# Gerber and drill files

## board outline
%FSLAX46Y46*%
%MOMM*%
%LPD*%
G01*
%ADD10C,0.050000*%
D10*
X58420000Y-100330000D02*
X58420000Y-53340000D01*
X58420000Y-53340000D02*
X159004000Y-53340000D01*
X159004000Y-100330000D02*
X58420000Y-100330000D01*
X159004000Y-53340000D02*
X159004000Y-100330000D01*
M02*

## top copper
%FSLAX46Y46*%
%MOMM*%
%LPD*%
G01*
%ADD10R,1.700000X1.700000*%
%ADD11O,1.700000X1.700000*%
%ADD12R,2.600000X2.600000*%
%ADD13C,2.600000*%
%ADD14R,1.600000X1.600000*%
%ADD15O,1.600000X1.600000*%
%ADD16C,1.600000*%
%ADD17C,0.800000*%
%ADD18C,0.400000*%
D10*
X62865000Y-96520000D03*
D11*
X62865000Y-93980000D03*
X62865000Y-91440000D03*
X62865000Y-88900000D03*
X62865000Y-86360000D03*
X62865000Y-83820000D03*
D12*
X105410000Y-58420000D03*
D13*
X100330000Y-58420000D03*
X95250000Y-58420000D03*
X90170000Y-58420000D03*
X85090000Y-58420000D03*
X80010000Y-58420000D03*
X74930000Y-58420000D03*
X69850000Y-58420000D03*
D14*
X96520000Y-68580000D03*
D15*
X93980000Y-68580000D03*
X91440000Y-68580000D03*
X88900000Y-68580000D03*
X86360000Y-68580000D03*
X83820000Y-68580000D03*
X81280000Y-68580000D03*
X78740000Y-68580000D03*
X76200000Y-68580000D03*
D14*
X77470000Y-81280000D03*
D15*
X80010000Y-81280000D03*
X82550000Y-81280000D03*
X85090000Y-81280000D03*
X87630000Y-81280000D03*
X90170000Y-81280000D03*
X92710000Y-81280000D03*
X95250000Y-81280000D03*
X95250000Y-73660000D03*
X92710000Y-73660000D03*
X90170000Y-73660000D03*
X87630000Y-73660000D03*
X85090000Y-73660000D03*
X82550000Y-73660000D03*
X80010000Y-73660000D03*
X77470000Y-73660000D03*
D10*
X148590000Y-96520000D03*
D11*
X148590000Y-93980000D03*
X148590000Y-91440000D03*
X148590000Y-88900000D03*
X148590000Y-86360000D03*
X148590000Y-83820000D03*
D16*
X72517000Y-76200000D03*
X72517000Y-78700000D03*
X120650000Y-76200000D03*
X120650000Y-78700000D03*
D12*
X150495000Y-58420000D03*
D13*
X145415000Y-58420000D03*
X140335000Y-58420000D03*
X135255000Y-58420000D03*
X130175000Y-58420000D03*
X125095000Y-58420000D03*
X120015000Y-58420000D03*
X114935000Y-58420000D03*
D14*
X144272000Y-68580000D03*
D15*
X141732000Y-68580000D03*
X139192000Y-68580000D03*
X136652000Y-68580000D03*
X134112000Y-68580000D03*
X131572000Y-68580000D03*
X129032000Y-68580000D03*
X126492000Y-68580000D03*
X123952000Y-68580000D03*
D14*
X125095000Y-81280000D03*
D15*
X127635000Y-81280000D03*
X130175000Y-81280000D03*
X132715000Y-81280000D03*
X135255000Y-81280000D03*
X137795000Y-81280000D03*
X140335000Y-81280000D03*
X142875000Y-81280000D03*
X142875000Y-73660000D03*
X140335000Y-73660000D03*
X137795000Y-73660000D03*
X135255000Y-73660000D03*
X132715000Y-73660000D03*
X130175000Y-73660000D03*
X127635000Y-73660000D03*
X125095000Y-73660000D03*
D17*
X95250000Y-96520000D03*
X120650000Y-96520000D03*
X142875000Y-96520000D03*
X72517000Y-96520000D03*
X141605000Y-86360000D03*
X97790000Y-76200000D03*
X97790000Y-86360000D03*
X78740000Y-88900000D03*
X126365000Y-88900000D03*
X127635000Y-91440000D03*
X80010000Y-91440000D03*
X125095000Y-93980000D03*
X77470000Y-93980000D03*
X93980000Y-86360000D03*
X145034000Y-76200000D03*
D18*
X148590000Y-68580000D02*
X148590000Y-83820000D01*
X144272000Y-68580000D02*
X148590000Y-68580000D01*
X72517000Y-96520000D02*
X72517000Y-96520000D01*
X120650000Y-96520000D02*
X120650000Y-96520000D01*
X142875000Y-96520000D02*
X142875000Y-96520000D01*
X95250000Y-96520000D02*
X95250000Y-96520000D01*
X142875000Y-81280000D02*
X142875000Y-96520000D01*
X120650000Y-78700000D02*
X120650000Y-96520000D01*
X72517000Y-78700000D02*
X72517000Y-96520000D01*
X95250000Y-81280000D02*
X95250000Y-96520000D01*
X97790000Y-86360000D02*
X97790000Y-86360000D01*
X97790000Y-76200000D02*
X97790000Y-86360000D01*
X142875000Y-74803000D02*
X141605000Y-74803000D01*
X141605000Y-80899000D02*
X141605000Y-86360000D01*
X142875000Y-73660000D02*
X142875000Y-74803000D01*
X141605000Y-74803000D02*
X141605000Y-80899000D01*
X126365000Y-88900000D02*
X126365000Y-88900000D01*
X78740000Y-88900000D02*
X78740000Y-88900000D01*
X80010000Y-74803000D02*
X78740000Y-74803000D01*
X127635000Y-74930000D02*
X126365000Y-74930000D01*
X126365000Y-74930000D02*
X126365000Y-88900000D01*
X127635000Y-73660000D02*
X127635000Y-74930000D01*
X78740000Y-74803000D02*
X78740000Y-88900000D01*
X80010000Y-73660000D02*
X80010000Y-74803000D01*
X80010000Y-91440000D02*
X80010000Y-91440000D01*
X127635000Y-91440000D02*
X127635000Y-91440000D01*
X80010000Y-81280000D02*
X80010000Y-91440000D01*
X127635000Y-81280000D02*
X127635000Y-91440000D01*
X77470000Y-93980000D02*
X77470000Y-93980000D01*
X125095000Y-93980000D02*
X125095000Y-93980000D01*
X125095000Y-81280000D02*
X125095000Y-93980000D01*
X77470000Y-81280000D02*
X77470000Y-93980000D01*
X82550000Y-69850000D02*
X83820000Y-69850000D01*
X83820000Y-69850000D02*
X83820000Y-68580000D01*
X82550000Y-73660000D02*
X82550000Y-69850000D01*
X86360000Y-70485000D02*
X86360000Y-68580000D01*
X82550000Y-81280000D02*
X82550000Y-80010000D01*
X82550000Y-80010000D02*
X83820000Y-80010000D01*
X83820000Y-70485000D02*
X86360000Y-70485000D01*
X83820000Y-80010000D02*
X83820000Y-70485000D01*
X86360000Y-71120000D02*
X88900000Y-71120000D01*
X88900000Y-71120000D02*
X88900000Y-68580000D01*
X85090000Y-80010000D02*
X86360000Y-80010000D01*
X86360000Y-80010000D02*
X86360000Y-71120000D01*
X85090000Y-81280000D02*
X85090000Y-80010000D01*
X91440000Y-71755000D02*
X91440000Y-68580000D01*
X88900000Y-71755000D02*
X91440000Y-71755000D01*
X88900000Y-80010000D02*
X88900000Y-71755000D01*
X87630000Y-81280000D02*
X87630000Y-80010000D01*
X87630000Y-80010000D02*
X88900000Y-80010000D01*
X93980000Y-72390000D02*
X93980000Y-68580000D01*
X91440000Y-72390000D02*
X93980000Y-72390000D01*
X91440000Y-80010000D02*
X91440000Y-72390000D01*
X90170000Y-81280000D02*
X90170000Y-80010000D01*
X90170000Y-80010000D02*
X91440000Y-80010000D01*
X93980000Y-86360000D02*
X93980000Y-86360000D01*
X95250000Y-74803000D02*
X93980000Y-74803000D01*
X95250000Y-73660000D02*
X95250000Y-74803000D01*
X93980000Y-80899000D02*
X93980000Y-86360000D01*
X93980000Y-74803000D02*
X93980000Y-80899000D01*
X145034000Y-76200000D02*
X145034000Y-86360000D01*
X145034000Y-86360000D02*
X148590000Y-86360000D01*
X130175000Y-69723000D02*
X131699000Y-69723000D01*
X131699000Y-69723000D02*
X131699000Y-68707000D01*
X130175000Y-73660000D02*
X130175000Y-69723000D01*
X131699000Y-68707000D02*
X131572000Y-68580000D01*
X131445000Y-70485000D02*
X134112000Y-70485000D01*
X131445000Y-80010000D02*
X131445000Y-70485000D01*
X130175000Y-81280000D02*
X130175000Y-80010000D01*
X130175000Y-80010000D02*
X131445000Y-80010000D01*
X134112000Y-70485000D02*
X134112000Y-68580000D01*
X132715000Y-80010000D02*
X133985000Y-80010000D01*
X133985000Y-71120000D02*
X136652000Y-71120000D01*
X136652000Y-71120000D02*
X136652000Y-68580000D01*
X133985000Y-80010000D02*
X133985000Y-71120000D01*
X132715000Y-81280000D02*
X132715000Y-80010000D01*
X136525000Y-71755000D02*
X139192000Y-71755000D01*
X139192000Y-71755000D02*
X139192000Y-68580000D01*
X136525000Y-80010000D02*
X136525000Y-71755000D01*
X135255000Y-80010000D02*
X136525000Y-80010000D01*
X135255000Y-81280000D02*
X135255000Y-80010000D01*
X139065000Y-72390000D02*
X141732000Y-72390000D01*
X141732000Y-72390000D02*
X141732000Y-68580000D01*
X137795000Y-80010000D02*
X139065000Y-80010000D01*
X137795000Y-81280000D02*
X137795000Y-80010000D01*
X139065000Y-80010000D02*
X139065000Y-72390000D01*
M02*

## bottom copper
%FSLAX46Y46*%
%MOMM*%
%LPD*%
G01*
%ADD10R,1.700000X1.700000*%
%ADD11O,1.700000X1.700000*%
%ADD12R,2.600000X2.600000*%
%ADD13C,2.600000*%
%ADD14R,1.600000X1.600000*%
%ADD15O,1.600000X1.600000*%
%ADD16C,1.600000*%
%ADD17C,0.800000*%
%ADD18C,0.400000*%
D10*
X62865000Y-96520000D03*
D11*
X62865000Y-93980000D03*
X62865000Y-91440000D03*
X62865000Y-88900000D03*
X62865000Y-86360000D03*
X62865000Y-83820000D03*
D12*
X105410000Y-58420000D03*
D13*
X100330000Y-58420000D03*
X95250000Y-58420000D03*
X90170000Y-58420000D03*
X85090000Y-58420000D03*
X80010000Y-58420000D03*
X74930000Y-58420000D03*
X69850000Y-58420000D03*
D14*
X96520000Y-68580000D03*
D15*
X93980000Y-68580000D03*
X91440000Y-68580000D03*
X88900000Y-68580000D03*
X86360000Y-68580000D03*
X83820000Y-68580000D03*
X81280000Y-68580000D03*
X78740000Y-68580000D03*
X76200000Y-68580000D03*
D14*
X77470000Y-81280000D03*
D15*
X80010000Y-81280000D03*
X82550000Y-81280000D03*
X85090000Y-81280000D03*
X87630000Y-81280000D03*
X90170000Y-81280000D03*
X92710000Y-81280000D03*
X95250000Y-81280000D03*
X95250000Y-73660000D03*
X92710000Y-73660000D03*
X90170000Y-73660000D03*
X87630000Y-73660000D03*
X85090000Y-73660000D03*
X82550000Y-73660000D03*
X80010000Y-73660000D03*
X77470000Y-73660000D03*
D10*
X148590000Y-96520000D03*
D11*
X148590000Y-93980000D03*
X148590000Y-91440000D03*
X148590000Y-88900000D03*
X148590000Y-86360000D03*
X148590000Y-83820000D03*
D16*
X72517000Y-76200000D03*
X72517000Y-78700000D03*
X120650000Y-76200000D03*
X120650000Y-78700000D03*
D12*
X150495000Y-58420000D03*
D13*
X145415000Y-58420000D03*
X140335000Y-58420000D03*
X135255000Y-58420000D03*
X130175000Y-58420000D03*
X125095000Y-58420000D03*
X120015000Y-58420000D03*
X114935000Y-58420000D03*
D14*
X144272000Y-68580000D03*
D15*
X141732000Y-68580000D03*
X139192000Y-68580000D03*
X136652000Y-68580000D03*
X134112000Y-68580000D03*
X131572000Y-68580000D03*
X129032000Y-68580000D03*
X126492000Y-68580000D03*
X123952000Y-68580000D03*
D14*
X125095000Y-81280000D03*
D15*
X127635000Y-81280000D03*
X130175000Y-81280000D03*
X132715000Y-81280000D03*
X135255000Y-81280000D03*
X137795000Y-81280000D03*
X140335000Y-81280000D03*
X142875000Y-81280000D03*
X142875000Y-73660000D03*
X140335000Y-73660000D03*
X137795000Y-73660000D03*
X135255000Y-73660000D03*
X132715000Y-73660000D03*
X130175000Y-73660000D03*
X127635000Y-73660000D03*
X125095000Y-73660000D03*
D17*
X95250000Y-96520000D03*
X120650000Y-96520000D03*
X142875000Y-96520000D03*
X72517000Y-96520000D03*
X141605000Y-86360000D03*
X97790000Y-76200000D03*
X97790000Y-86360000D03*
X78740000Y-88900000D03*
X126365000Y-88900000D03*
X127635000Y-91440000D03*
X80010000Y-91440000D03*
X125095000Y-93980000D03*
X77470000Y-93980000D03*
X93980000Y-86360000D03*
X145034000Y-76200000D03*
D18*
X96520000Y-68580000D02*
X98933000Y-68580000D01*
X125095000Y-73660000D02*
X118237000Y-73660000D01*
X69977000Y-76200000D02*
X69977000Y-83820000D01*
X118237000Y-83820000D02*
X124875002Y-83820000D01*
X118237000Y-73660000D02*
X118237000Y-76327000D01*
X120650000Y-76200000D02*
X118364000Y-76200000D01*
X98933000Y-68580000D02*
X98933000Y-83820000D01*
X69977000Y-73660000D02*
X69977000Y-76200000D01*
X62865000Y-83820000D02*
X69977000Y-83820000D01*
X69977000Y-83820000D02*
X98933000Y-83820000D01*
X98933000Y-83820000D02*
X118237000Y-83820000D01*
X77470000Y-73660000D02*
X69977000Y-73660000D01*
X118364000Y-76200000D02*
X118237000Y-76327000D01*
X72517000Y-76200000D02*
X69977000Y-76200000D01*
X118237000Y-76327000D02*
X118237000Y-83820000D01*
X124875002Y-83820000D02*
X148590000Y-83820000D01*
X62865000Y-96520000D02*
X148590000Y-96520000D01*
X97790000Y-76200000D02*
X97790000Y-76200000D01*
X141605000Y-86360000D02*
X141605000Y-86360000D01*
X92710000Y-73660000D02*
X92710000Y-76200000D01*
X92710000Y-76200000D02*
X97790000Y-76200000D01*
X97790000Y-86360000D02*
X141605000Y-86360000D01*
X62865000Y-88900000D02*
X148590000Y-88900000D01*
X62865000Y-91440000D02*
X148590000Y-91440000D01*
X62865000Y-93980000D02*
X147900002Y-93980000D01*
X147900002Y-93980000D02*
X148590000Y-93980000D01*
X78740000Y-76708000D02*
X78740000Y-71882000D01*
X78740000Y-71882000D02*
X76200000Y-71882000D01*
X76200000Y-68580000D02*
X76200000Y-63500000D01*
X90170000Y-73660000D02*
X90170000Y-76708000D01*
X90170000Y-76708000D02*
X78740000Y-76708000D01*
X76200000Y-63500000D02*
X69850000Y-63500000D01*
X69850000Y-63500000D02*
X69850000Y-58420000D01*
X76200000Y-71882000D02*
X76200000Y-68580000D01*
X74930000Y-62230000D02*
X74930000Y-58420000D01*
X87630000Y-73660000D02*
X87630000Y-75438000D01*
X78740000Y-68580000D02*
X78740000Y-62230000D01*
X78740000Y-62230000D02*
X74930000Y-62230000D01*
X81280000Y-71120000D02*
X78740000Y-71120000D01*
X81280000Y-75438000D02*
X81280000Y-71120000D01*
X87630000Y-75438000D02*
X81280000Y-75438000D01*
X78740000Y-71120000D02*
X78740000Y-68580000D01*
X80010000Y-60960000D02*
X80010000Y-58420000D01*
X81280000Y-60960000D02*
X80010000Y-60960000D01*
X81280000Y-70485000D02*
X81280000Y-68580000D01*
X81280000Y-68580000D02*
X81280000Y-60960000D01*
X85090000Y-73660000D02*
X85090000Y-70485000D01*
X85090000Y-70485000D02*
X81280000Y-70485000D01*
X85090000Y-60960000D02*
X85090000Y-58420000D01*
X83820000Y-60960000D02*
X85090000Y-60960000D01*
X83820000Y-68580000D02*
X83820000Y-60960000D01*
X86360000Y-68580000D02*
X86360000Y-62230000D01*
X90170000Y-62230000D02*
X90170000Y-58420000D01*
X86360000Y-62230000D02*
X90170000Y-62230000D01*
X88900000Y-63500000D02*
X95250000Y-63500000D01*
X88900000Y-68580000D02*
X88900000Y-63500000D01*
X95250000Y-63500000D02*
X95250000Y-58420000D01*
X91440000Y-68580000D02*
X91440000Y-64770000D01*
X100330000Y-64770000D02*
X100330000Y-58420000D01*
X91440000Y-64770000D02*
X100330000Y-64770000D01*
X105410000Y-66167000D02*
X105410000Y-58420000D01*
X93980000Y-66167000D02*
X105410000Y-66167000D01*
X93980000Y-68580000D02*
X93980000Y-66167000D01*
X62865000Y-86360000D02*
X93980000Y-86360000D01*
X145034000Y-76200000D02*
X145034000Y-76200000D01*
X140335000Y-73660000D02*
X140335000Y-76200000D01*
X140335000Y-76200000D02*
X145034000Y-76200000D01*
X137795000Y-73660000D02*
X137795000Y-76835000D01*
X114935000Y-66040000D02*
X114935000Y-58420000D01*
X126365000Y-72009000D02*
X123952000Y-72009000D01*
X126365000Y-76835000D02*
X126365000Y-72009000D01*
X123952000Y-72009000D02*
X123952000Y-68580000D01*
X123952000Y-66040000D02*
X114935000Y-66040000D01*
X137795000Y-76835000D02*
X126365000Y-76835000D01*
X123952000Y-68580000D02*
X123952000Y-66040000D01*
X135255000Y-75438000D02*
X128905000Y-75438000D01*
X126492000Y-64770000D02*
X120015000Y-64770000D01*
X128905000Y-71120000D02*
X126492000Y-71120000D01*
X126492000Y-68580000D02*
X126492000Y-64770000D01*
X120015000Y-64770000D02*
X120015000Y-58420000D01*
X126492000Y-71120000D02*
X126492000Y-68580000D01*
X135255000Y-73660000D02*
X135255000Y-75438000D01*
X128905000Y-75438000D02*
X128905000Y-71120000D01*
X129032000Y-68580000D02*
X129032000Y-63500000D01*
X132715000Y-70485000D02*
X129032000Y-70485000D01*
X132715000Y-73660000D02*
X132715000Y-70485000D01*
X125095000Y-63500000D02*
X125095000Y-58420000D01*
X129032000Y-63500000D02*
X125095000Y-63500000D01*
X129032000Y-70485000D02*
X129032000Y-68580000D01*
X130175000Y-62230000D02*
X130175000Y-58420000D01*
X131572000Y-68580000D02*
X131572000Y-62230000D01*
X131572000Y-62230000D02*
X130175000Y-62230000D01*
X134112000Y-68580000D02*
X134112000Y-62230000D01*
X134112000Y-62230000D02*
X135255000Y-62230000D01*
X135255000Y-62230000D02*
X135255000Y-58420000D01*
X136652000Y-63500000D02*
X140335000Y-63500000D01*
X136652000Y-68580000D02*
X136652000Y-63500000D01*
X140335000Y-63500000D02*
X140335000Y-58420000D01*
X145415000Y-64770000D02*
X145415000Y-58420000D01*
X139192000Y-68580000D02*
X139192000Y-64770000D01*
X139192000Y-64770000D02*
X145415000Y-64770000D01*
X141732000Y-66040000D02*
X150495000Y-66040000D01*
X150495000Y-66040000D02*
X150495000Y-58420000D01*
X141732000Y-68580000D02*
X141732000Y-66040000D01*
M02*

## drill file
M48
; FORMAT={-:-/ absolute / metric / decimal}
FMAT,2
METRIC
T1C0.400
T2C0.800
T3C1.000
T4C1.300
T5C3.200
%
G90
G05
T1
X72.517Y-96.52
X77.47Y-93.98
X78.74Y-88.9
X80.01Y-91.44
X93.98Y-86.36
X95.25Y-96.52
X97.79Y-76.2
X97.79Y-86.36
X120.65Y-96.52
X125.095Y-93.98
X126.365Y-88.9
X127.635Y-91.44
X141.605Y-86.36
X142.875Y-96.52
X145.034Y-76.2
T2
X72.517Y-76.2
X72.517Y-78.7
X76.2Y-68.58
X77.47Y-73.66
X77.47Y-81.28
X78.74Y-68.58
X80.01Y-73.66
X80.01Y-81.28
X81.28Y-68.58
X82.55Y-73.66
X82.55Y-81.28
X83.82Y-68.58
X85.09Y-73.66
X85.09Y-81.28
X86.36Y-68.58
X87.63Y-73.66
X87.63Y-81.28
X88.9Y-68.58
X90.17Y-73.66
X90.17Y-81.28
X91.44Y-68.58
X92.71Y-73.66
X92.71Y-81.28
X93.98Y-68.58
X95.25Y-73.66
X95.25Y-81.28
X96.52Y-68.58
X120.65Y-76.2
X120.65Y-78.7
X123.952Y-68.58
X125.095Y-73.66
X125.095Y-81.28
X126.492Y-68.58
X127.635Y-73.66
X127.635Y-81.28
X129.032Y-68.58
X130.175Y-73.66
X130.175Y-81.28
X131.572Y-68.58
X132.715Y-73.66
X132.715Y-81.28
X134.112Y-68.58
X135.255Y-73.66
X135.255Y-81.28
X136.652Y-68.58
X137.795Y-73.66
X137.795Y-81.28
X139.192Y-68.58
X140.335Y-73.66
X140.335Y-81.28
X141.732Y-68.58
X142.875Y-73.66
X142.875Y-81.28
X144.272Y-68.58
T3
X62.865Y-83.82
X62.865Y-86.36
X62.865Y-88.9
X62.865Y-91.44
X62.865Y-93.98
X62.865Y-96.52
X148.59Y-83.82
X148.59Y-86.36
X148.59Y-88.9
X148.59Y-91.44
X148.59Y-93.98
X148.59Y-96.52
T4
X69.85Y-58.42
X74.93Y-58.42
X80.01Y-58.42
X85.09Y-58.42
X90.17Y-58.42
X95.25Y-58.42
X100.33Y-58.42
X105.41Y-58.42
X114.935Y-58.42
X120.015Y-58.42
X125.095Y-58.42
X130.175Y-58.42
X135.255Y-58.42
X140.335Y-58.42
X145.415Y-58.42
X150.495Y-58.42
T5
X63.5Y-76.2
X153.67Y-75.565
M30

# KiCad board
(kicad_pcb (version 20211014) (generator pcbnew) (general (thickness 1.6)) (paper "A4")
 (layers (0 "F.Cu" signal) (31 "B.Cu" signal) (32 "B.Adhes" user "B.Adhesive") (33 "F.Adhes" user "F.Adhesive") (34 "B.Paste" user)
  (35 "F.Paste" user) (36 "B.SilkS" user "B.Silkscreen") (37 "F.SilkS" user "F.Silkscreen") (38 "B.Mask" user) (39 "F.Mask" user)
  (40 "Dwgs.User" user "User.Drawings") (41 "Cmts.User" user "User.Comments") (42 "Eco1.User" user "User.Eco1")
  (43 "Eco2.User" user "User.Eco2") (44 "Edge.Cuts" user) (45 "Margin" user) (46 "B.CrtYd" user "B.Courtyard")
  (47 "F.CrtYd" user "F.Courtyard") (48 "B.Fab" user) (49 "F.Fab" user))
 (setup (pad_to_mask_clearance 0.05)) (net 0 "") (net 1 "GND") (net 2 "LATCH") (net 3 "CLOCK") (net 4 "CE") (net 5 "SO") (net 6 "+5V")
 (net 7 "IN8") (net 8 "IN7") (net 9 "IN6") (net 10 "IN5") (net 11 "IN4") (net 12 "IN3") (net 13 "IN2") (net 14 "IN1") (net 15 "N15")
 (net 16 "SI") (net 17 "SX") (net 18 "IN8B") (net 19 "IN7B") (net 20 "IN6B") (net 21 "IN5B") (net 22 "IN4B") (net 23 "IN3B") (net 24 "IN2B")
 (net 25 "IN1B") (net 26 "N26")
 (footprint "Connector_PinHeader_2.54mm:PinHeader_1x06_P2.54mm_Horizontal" (layer "F.Cu") (at 62.865 96.52 180)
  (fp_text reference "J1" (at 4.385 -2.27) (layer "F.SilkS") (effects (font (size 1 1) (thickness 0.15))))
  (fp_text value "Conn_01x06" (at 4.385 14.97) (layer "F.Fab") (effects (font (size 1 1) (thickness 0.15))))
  (pad "1" thru_hole rect locked (at 0 0 180) (size 1.7 1.7) (drill 1) (layers *.Cu *.Mask) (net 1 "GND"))
  (pad "2" thru_hole oval locked (at 0 2.54 180) (size 1.7 1.7) (drill 1) (layers *.Cu *.Mask) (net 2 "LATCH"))
  (pad "3" thru_hole oval locked (at 0 5.08 180) (size 1.7 1.7) (drill 1) (layers *.Cu *.Mask) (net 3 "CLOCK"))
  (pad "4" thru_hole oval locked (at 0 7.62 180) (size 1.7 1.7) (drill 1) (layers *.Cu *.Mask) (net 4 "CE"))
  (pad "5" thru_hole oval locked (at 0 10.16 180) (size 1.7 1.7) (drill 1) (layers *.Cu *.Mask) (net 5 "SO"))
  (pad "6" thru_hole oval locked (at 0 12.7 180) (size 1.7 1.7) (drill 1) (layers *.Cu *.Mask) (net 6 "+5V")))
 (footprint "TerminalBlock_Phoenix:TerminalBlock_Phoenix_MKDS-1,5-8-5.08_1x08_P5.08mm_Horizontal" (layer "F.Cu") (at 105.41 58.42 180)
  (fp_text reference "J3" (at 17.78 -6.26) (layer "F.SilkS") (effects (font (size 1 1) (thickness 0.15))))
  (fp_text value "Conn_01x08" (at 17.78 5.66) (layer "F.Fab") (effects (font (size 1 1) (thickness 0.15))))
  (pad "1" thru_hole rect locked (at 0 0 180) (size 2.6 2.6) (drill 1.3) (layers *.Cu *.Mask) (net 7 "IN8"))
  (pad "2" thru_hole circle locked (at 5.08 0 180) (size 2.6 2.6) (drill 1.3) (layers *.Cu *.Mask) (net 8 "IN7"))
  (pad "3" thru_hole circle locked (at 10.16 0 180) (size 2.6 2.6) (drill 1.3) (layers *.Cu *.Mask) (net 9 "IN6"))
  (pad "4" thru_hole circle locked (at 15.24 0 180) (size 2.6 2.6) (drill 1.3) (layers *.Cu *.Mask) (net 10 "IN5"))
  (pad "5" thru_hole circle locked (at 20.32 0 180) (size 2.6 2.6) (drill 1.3) (layers *.Cu *.Mask) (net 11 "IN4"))
  (pad "6" thru_hole circle locked (at 25.4 0 180) (size 2.6 2.6) (drill 1.3) (layers *.Cu *.Mask) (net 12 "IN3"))
  (pad "7" thru_hole circle locked (at 30.48 0 180) (size 2.6 2.6) (drill 1.3) (layers *.Cu *.Mask) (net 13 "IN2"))
  (pad "8" thru_hole circle locked (at 35.56 0 180) (size 2.6 2.6) (drill 1.3) (layers *.Cu *.Mask) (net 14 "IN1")))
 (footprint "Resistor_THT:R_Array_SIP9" (layer "F.Cu") (at 96.52 68.58 180)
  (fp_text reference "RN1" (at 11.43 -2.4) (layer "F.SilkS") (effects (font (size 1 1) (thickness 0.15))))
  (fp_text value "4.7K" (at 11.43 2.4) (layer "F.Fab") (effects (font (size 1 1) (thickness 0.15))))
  (pad "1" thru_hole rect locked (at 0 0 180) (size 1.6 1.6) (drill 0.8) (layers *.Cu *.Mask) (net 6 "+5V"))
  (pad "2" thru_hole oval locked (at 2.54 0 180) (size 1.6 1.6) (drill 0.8) (layers *.Cu *.Mask) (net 7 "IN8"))
  (pad "3" thru_hole oval locked (at 5.08 0 180) (size 1.6 1.6) (drill 0.8) (layers *.Cu *.Mask) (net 8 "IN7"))
  (pad "4" thru_hole oval locked (at 7.62 0 180) (size 1.6 1.6) (drill 0.8) (layers *.Cu *.Mask) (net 9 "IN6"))
  (pad "5" thru_hole oval locked (at 10.16 0 180) (size 1.6 1.6) (drill 0.8) (layers *.Cu *.Mask) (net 10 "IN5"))
  (pad "6" thru_hole oval locked (at 12.7 0 180) (size 1.6 1.6) (drill 0.8) (layers *.Cu *.Mask) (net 11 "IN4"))
  (pad "7" thru_hole oval locked (at 15.24 0 180) (size 1.6 1.6) (drill 0.8) (layers *.Cu *.Mask) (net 12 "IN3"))
  (pad "8" thru_hole oval locked (at 17.78 0 180) (size 1.6 1.6) (drill 0.8) (layers *.Cu *.Mask) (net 13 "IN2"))
  (pad "9" thru_hole oval locked (at 20.32 0 180) (size 1.6 1.6) (drill 0.8) (layers *.Cu *.Mask) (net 14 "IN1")))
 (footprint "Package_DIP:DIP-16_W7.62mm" (layer "F.Cu") (at 77.47 81.28 90)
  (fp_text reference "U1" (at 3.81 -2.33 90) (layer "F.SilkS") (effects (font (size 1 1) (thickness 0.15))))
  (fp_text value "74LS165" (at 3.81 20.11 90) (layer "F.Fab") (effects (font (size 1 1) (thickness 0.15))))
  (pad "1" thru_hole rect locked (at 0 0 90) (size 1.6 1.6) (drill 0.8) (layers *.Cu *.Mask) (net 2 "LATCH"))
  (pad "2" thru_hole oval locked (at 0 2.54 90) (size 1.6 1.6) (drill 0.8) (layers *.Cu *.Mask) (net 3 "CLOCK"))
  (pad "3" thru_hole oval locked (at 0 5.08 90) (size 1.6 1.6) (drill 0.8) (layers *.Cu *.Mask) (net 10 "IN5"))
  (pad "4" thru_hole oval locked (at 0 7.62 90) (size 1.6 1.6) (drill 0.8) (layers *.Cu *.Mask) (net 9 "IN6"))
  (pad "5" thru_hole oval locked (at 0 10.16 90) (size 1.6 1.6) (drill 0.8) (layers *.Cu *.Mask) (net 8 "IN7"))
  (pad "6" thru_hole oval locked (at 0 12.7 90) (size 1.6 1.6) (drill 0.8) (layers *.Cu *.Mask) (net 7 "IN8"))
  (pad "7" thru_hole oval locked (at 0 15.24 90) (size 1.6 1.6) (drill 0.8) (layers *.Cu *.Mask) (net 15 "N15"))
  (pad "8" thru_hole oval locked (at 0 17.78 90) (size 1.6 1.6) (drill 0.8) (layers *.Cu *.Mask) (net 1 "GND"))
  (pad "9" thru_hole oval locked (at 7.62 17.78 90) (size 1.6 1.6) (drill 0.8) (layers *.Cu *.Mask) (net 5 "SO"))
  (pad "10" thru_hole oval locked (at 7.62 15.24 90) (size 1.6 1.6) (drill 0.8) (layers *.Cu *.Mask) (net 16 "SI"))
  (pad "11" thru_hole oval locked (at 7.62 12.7 90) (size 1.6 1.6) (drill 0.8) (layers *.Cu *.Mask) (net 14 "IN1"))
  (pad "12" thru_hole oval locked (at 7.62 10.16 90) (size 1.6 1.6) (drill 0.8) (layers *.Cu *.Mask) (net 13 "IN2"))
  (pad "13" thru_hole oval locked (at 7.62 7.62 90) (size 1.6 1.6) (drill 0.8) (layers *.Cu *.Mask) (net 12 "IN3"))
  (pad "14" thru_hole oval locked (at 7.62 5.08 90) (size 1.6 1.6) (drill 0.8) (layers *.Cu *.Mask) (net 11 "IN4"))
  (pad "15" thru_hole oval locked (at 7.62 2.54 90) (size 1.6 1.6) (drill 0.8) (layers *.Cu *.Mask) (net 4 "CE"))
  (pad "16" thru_hole oval locked (at 7.62 0 90) (size 1.6 1.6) (drill 0.8) (layers *.Cu *.Mask) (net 6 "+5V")))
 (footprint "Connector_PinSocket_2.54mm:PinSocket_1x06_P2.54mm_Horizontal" (layer "F.Cu") (at 148.59 96.52 180)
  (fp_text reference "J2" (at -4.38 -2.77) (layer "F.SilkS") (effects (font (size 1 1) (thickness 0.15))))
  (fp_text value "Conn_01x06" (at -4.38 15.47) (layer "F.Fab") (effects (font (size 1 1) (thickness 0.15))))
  (pad "1" thru_hole rect locked (at 0 0 180) (size 1.7 1.7) (drill 1) (layers *.Cu *.Mask) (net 1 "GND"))
  (pad "2" thru_hole oval locked (at 0 2.54 180) (size 1.7 1.7) (drill 1) (layers *.Cu *.Mask) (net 2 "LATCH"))
  (pad "3" thru_hole oval locked (at 0 5.08 180) (size 1.7 1.7) (drill 1) (layers *.Cu *.Mask) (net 3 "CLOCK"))
  (pad "4" thru_hole oval locked (at 0 7.62 180) (size 1.7 1.7) (drill 1) (layers *.Cu *.Mask) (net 4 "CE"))
  (pad "5" thru_hole oval locked (at 0 10.16 180) (size 1.7 1.7) (drill 1) (layers *.Cu *.Mask) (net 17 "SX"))
  (pad "6" thru_hole oval locked (at 0 12.7 180) (size 1.7 1.7) (drill 1) (layers *.Cu *.Mask) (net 6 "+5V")))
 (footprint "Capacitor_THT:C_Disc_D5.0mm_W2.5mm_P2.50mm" (layer "F.Cu") (at 72.517 76.2 -90)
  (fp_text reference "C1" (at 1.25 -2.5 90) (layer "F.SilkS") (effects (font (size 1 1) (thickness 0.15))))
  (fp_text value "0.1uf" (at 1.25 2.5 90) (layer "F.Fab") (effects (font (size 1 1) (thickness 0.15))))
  (pad "1" thru_hole circle locked (at 0 0 270) (size 1.6 1.6) (drill 0.8) (layers *.Cu *.Mask) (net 6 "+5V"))
  (pad "2" thru_hole circle locked (at 2.5 0 270) (size 1.6 1.6) (drill 0.8) (layers *.Cu *.Mask) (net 1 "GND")))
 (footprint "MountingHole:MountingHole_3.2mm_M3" (layer "F.Cu") (at 153.67 75.565)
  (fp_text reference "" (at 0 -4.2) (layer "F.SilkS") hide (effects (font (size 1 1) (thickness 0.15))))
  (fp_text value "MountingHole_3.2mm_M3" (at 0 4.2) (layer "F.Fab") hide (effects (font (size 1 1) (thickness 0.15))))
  (pad "" np_thru_hole circle locked (at 0 0) (size 3.2 3.2) (drill 3.2) (layers *.Cu *.Mask)))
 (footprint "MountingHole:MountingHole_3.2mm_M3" (layer "F.Cu") (at 63.5 76.2)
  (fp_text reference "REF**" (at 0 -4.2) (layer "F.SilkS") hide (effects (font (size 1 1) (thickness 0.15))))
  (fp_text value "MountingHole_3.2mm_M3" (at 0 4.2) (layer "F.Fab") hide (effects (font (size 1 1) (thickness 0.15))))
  (pad "" np_thru_hole circle locked (at 0 0) (size 3.2 3.2) (drill 3.2) (layers *.Cu *.Mask)))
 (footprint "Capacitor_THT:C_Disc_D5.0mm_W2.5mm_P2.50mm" (layer "F.Cu") (at 120.65 76.2 -90)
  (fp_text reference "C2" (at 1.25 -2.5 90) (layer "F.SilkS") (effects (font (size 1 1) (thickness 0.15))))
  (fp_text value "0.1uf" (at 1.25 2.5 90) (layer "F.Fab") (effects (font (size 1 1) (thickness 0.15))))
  (pad "1" thru_hole circle locked (at 0 0 270) (size 1.6 1.6) (drill 0.8) (layers *.Cu *.Mask) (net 6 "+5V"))
  (pad "2" thru_hole circle locked (at 2.5 0 270) (size 1.6 1.6) (drill 0.8) (layers *.Cu *.Mask) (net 1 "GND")))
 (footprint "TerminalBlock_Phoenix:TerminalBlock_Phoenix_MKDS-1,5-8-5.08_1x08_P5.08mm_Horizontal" (layer "F.Cu") (at 150.495 58.42 180)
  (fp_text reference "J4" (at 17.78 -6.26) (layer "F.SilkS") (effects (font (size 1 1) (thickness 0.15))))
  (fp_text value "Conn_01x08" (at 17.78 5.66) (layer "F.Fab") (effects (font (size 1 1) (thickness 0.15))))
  (pad "1" thru_hole rect locked (at 0 0 180) (size 2.6 2.6) (drill 1.3) (layers *.Cu *.Mask) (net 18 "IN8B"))
  (pad "2" thru_hole circle locked (at 5.08 0 180) (size 2.6 2.6) (drill 1.3) (layers *.Cu *.Mask) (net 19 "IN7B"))
  (pad "3" thru_hole circle locked (at 10.16 0 180) (size 2.6 2.6) (drill 1.3) (layers *.Cu *.Mask) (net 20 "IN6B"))
  (pad "4" thru_hole circle locked (at 15.24 0 180) (size 2.6 2.6) (drill 1.3) (layers *.Cu *.Mask) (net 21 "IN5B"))
  (pad "5" thru_hole circle locked (at 20.32 0 180) (size 2.6 2.6) (drill 1.3) (layers *.Cu *.Mask) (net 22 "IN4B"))
  (pad "6" thru_hole circle locked (at 25.4 0 180) (size 2.6 2.6) (drill 1.3) (layers *.Cu *.Mask) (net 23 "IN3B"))
  (pad "7" thru_hole circle locked (at 30.48 0 180) (size 2.6 2.6) (drill 1.3) (layers *.Cu *.Mask) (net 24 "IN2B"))
  (pad "8" thru_hole circle locked (at 35.56 0 180) (size 2.6 2.6) (drill 1.3) (layers *.Cu *.Mask) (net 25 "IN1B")))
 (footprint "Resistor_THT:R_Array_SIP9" (layer "F.Cu") (at 144.272 68.58 180)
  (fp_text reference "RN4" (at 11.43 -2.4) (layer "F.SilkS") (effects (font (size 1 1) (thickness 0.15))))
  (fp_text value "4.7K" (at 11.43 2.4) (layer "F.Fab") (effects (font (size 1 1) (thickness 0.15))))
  (pad "1" thru_hole rect locked (at 0 0 180) (size 1.6 1.6) (drill 0.8) (layers *.Cu *.Mask) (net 6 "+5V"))
  (pad "2" thru_hole oval locked (at 2.54 0 180) (size 1.6 1.6) (drill 0.8) (layers *.Cu *.Mask) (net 18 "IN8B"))
  (pad "3" thru_hole oval locked (at 5.08 0 180) (size 1.6 1.6) (drill 0.8) (layers *.Cu *.Mask) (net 19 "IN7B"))
  (pad "4" thru_hole oval locked (at 7.62 0 180) (size 1.6 1.6) (drill 0.8) (layers *.Cu *.Mask) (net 20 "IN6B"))
  (pad "5" thru_hole oval locked (at 10.16 0 180) (size 1.6 1.6) (drill 0.8) (layers *.Cu *.Mask) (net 21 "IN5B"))
  (pad "6" thru_hole oval locked (at 12.7 0 180) (size 1.6 1.6) (drill 0.8) (layers *.Cu *.Mask) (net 22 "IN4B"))
  (pad "7" thru_hole oval locked (at 15.24 0 180) (size 1.6 1.6) (drill 0.8) (layers *.Cu *.Mask) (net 23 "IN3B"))
  (pad "8" thru_hole oval locked (at 17.78 0 180) (size 1.6 1.6) (drill 0.8) (layers *.Cu *.Mask) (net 24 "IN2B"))
  (pad "9" thru_hole oval locked (at 20.32 0 180) (size 1.6 1.6) (drill 0.8) (layers *.Cu *.Mask) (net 25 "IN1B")))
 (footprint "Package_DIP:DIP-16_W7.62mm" (layer "F.Cu") (at 125.095 81.28 90)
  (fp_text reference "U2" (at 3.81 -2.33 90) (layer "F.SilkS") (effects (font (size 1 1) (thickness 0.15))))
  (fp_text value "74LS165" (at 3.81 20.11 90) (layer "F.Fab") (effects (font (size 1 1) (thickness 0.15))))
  (pad "1" thru_hole rect locked (at 0 0 90) (size 1.6 1.6) (drill 0.8) (layers *.Cu *.Mask) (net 2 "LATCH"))
  (pad "2" thru_hole oval locked (at 0 2.54 90) (size 1.6 1.6) (drill 0.8) (layers *.Cu *.Mask) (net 3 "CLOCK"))
  (pad "3" thru_hole oval locked (at 0 5.08 90) (size 1.6 1.6) (drill 0.8) (layers *.Cu *.Mask) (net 21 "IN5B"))
  (pad "4" thru_hole oval locked (at 0 7.62 90) (size 1.6 1.6) (drill 0.8) (layers *.Cu *.Mask) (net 20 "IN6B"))
  (pad "5" thru_hole oval locked (at 0 10.16 90) (size 1.6 1.6) (drill 0.8) (layers *.Cu *.Mask) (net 19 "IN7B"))
  (pad "6" thru_hole oval locked (at 0 12.7 90) (size 1.6 1.6) (drill 0.8) (layers *.Cu *.Mask) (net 18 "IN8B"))
  (pad "7" thru_hole oval locked (at 0 15.24 90) (size 1.6 1.6) (drill 0.8) (layers *.Cu *.Mask) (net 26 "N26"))
  (pad "8" thru_hole oval locked (at 0 17.78 90) (size 1.6 1.6) (drill 0.8) (layers *.Cu *.Mask) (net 1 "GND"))
  (pad "9" thru_hole oval locked (at 7.62 17.78 90) (size 1.6 1.6) (drill 0.8) (layers *.Cu *.Mask) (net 16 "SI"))
  (pad "10" thru_hole oval locked (at 7.62 15.24 90) (size 1.6 1.6) (drill 0.8) (layers *.Cu *.Mask) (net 17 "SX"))
  (pad "11" thru_hole oval locked (at 7.62 12.7 90) (size 1.6 1.6) (drill 0.8) (layers *.Cu *.Mask) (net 25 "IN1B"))
  (pad "12" thru_hole oval locked (at 7.62 10.16 90) (size 1.6 1.6) (drill 0.8) (layers *.Cu *.Mask) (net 24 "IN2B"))
  (pad "13" thru_hole oval locked (at 7.62 7.62 90) (size 1.6 1.6) (drill 0.8) (layers *.Cu *.Mask) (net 23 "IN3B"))
  (pad "14" thru_hole oval locked (at 7.62 5.08 90) (size 1.6 1.6) (drill 0.8) (layers *.Cu *.Mask) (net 22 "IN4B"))
  (pad "15" thru_hole oval locked (at 7.62 2.54 90) (size 1.6 1.6) (drill 0.8) (layers *.Cu *.Mask) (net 4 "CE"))
  (pad "16" thru_hole oval locked (at 7.62 0 90) (size 1.6 1.6) (drill 0.8) (layers *.Cu *.Mask) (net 6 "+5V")))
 (gr_line (start 58.42 100.33) (end 58.42 53.34) (layer "Edge.Cuts") (width 0.05))
 (gr_line (start 58.42 53.34) (end 159.004 53.34) (layer "Edge.Cuts") (width 0.05))
 (gr_line (start 159.004 100.33) (end 58.42 100.33) (layer "Edge.Cuts") (width 0.05))
 (gr_line (start 159.004 53.34) (end 159.004 100.33) (layer "Edge.Cuts") (width 0.05))
 (segment (start 148.59 68.58) (end 148.59 83.82) (width 0.4) (layer "F.Cu") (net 6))
 (segment (start 144.272 68.58) (end 148.59 68.58) (width 0.4) (layer "F.Cu") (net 6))
 (segment (start 96.52 68.58) (end 98.933 68.58) (width 0.4) (layer "B.Cu") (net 6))
 (segment (start 125.095 73.66) (end 118.237 73.66) (width 0.4) (layer "B.Cu") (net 6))
 (segment (start 69.977 76.2) (end 69.977 83.82) (width 0.4) (layer "B.Cu") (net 6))
 (segment (start 118.237 83.82) (end 124.875002 83.82) (width 0.4) (layer "B.Cu") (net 6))
 (segment (start 118.237 73.66) (end 118.237 76.327) (width 0.4) (layer "B.Cu") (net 6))
 (segment (start 120.65 76.2) (end 118.364 76.2) (width 0.4) (layer "B.Cu") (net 6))
 (segment (start 98.933 68.58) (end 98.933 83.82) (width 0.4) (layer "B.Cu") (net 6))
 (segment (start 69.977 73.66) (end 69.977 76.2) (width 0.4) (layer "B.Cu") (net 6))
 (segment (start 62.865 83.82) (end 69.977 83.82) (width 0.4) (layer "B.Cu") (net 6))
 (segment (start 69.977 83.82) (end 98.933 83.82) (width 0.4) (layer "B.Cu") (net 6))
 (segment (start 98.933 83.82) (end 118.237 83.82) (width 0.4) (layer "B.Cu") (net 6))
 (segment (start 77.47 73.66) (end 69.977 73.66) (width 0.4) (layer "B.Cu") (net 6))
 (segment (start 118.364 76.2) (end 118.237 76.327) (width 0.4) (layer "B.Cu") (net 6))
 (segment (start 72.517 76.2) (end 69.977 76.2) (width 0.4) (layer "B.Cu") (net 6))
 (segment (start 118.237 76.327) (end 118.237 83.82) (width 0.4) (layer "B.Cu") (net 6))
 (segment (start 124.875002 83.82) (end 148.59 83.82) (width 0.4) (layer "B.Cu") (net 6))
 (segment (start 72.517 96.52) (end 72.517 96.52) (width 0.4) (layer "F.Cu") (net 1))
 (segment (start 120.65 96.52) (end 120.65 96.52) (width 0.4) (layer "F.Cu") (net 1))
 (segment (start 142.875 96.52) (end 142.875 96.52) (width 0.4) (layer "F.Cu") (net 1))
 (segment (start 95.25 96.52) (end 95.25 96.52) (width 0.4) (layer "F.Cu") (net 1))
 (segment (start 142.875 81.28) (end 142.875 96.52) (width 0.4) (layer "F.Cu") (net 1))
 (segment (start 120.65 78.7) (end 120.65 96.52) (width 0.4) (layer "F.Cu") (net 1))
 (segment (start 72.517 78.7) (end 72.517 96.52) (width 0.4) (layer "F.Cu") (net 1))
 (segment (start 95.25 81.28) (end 95.25 96.52) (width 0.4) (layer "F.Cu") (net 1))
 (via (at 95.25 96.52) (size 0.8) (drill 0.4) (layers "F.Cu" "B.Cu") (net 1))
 (via (at 120.65 96.52) (size 0.8) (drill 0.4) (layers "F.Cu" "B.Cu") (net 1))
 (via (at 142.875 96.52) (size 0.8) (drill 0.4) (layers "F.Cu" "B.Cu") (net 1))
 (via (at 72.517 96.52) (size 0.8) (drill 0.4) (layers "F.Cu" "B.Cu") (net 1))
 (segment (start 62.865 96.52) (end 148.59 96.52) (width 0.4) (layer "B.Cu") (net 1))
 (segment (start 97.79 86.36) (end 97.79 86.36) (width 0.4) (layer "F.Cu") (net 16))
 (segment (start 97.79 76.2) (end 97.79 86.36) (width 0.4) (layer "F.Cu") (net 16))
 (segment (start 142.875 74.803) (end 141.605 74.803) (width 0.4) (layer "F.Cu") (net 16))
 (segment (start 141.605 80.899) (end 141.605 86.36) (width 0.4) (layer "F.Cu") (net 16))
 (segment (start 142.875 73.66) (end 142.875 74.803) (width 0.4) (layer "F.Cu") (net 16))
 (segment (start 141.605 74.803) (end 141.605 80.899) (width 0.4) (layer "F.Cu") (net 16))
 (via (at 141.605 86.36) (size 0.8) (drill 0.4) (layers "F.Cu" "B.Cu") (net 16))
 (via (at 97.79 76.2) (size 0.8) (drill 0.4) (layers "F.Cu" "B.Cu") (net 16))
 (via (at 97.79 86.36) (size 0.8) (drill 0.4) (layers "F.Cu" "B.Cu") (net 16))
 (segment (start 97.79 76.2) (end 97.79 76.2) (width 0.4) (layer "B.Cu") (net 16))
 (segment (start 141.605 86.36) (end 141.605 86.36) (width 0.4) (layer "B.Cu") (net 16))
 (segment (start 92.71 73.66) (end 92.71 76.2) (width 0.4) (layer "B.Cu") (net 16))
 (segment (start 92.71 76.2) (end 97.79 76.2) (width 0.4) (layer "B.Cu") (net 16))
 (segment (start 97.79 86.36) (end 141.605 86.36) (width 0.4) (layer "B.Cu") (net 16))
 (segment (start 126.365 88.9) (end 126.365 88.9) (width 0.4) (layer "F.Cu") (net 4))
 (segment (start 78.74 88.9) (end 78.74 88.9) (width 0.4) (layer "F.Cu") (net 4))
 (segment (start 80.01 74.803) (end 78.74 74.803) (width 0.4) (layer "F.Cu") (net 4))
 (segment (start 127.635 74.93) (end 126.365 74.93) (width 0.4) (layer "F.Cu") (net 4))
 (segment (start 126.365 74.93) (end 126.365 88.9) (width 0.4) (layer "F.Cu") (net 4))
 (segment (start 127.635 73.66) (end 127.635 74.93) (width 0.4) (layer "F.Cu") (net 4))
 (segment (start 78.74 74.803) (end 78.74 88.9) (width 0.4) (layer "F.Cu") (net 4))
 (segment (start 80.01 73.66) (end 80.01 74.803) (width 0.4) (layer "F.Cu") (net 4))
 (via (at 78.74 88.9) (size 0.8) (drill 0.4) (layers "F.Cu" "B.Cu") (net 4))
 (via (at 126.365 88.9) (size 0.8) (drill 0.4) (layers "F.Cu" "B.Cu") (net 4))
 (segment (start 62.865 88.9) (end 148.59 88.9) (width 0.4) (layer "B.Cu") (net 4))
 (segment (start 80.01 91.44) (end 80.01 91.44) (width 0.4) (layer "F.Cu") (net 3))
 (segment (start 127.635 91.44) (end 127.635 91.44) (width 0.4) (layer "F.Cu") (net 3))
 (segment (start 80.01 81.28) (end 80.01 91.44) (width 0.4) (layer "F.Cu") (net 3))
 (segment (start 127.635 81.28) (end 127.635 91.44) (width 0.4) (layer "F.Cu") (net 3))
 (via (at 127.635 91.44) (size 0.8) (drill 0.4) (layers "F.Cu" "B.Cu") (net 3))
 (via (at 80.01 91.44) (size 0.8) (drill 0.4) (layers "F.Cu" "B.Cu") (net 3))
 (segment (start 62.865 91.44) (end 148.59 91.44) (width 0.4) (layer "B.Cu") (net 3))
 (segment (start 77.47 93.98) (end 77.47 93.98) (width 0.4) (layer "F.Cu") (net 2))
 (segment (start 125.095 93.98) (end 125.095 93.98) (width 0.4) (layer "F.Cu") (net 2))
 (segment (start 125.095 81.28) (end 125.095 93.98) (width 0.4) (layer "F.Cu") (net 2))
 (segment (start 77.47 81.28) (end 77.47 93.98) (width 0.4) (layer "F.Cu") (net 2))
 (via (at 125.095 93.98) (size 0.8) (drill 0.4) (layers "F.Cu" "B.Cu") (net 2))
 (via (at 77.47 93.98) (size 0.8) (drill 0.4) (layers "F.Cu" "B.Cu") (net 2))
 (segment (start 62.865 93.98) (end 147.900002 93.98) (width 0.4) (layer "B.Cu") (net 2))
 (segment (start 147.900002 93.98) (end 148.59 93.98) (width 0.4) (layer "B.Cu") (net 2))
 (segment (start 78.74 76.708) (end 78.74 71.882) (width 0.4) (layer "B.Cu") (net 14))
 (segment (start 78.74 71.882) (end 76.2 71.882) (width 0.4) (layer "B.Cu") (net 14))
 (segment (start 76.2 68.58) (end 76.2 63.5) (width 0.4) (layer "B.Cu") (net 14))
 (segment (start 90.17 73.66) (end 90.17 76.708) (width 0.4) (layer "B.Cu") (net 14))
 (segment (start 90.17 76.708) (end 78.74 76.708) (width 0.4) (layer "B.Cu") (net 14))
 (segment (start 76.2 63.5) (end 69.85 63.5) (width 0.4) (layer "B.Cu") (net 14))
 (segment (start 69.85 63.5) (end 69.85 58.42) (width 0.4) (layer "B.Cu") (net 14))
 (segment (start 76.2 71.882) (end 76.2 68.58) (width 0.4) (layer "B.Cu") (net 14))
 (segment (start 74.93 62.23) (end 74.93 58.42) (width 0.4) (layer "B.Cu") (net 13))
 (segment (start 87.63 73.66) (end 87.63 75.438) (width 0.4) (layer "B.Cu") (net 13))
 (segment (start 78.74 68.58) (end 78.74 62.23) (width 0.4) (layer "B.Cu") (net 13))
 (segment (start 78.74 62.23) (end 74.93 62.23) (width 0.4) (layer "B.Cu") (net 13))
 (segment (start 81.28 71.12) (end 78.74 71.12) (width 0.4) (layer "B.Cu") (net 13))
 (segment (start 81.28 75.438) (end 81.28 71.12) (width 0.4) (layer "B.Cu") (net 13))
 (segment (start 87.63 75.438) (end 81.28 75.438) (width 0.4) (layer "B.Cu") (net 13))
 (segment (start 78.74 71.12) (end 78.74 68.58) (width 0.4) (layer "B.Cu") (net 13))
 (segment (start 80.01 60.96) (end 80.01 58.42) (width 0.4) (layer "B.Cu") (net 12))
 (segment (start 81.28 60.96) (end 80.01 60.96) (width 0.4) (layer "B.Cu") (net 12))
 (segment (start 81.28 70.485) (end 81.28 68.58) (width 0.4) (layer "B.Cu") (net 12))
 (segment (start 81.28 68.58) (end 81.28 60.96) (width 0.4) (layer "B.Cu") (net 12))
 (segment (start 85.09 73.66) (end 85.09 70.485) (width 0.4) (layer "B.Cu") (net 12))
 (segment (start 85.09 70.485) (end 81.28 70.485) (width 0.4) (layer "B.Cu") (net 12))
 (segment (start 82.55 69.85) (end 83.82 69.85) (width 0.4) (layer "F.Cu") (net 11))
 (segment (start 83.82 69.85) (end 83.82 68.58) (width 0.4) (layer "F.Cu") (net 11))
 (segment (start 82.55 73.66) (end 82.55 69.85) (width 0.4) (layer "F.Cu") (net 11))
 (segment (start 85.09 60.96) (end 85.09 58.42) (width 0.4) (layer "B.Cu") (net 11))
 (segment (start 83.82 60.96) (end 85.09 60.96) (width 0.4) (layer "B.Cu") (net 11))
 (segment (start 83.82 68.58) (end 83.82 60.96) (width 0.4) (layer "B.Cu") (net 11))
 (segment (start 86.36 70.485) (end 86.36 68.58) (width 0.4) (layer "F.Cu") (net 10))
 (segment (start 82.55 81.28) (end 82.55 80.01) (width 0.4) (layer "F.Cu") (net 10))
 (segment (start 82.55 80.01) (end 83.82 80.01) (width 0.4) (layer "F.Cu") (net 10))
 (segment (start 83.82 70.485) (end 86.36 70.485) (width 0.4) (layer "F.Cu") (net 10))
 (segment (start 83.82 80.01) (end 83.82 70.485) (width 0.4) (layer "F.Cu") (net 10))
 (segment (start 86.36 68.58) (end 86.36 62.23) (width 0.4) (layer "B.Cu") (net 10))
 (segment (start 90.17 62.23) (end 90.17 58.42) (width 0.4) (layer "B.Cu") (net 10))
 (segment (start 86.36 62.23) (end 90.17 62.23) (width 0.4) (layer "B.Cu") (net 10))
 (segment (start 86.36 71.12) (end 88.9 71.12) (width 0.4) (layer "F.Cu") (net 9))
 (segment (start 88.9 71.12) (end 88.9 68.58) (width 0.4) (layer "F.Cu") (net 9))
 (segment (start 85.09 80.01) (end 86.36 80.01) (width 0.4) (layer "F.Cu") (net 9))
 (segment (start 86.36 80.01) (end 86.36 71.12) (width 0.4) (layer "F.Cu") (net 9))
 (segment (start 85.09 81.28) (end 85.09 80.01) (width 0.4) (layer "F.Cu") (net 9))
 (segment (start 88.9 63.5) (end 95.25 63.5) (width 0.4) (layer "B.Cu") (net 9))
 (segment (start 88.9 68.58) (end 88.9 63.5) (width 0.4) (layer "B.Cu") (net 9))
 (segment (start 95.25 63.5) (end 95.25 58.42) (width 0.4) (layer "B.Cu") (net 9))
 (segment (start 91.44 71.755) (end 91.44 68.58) (width 0.4) (layer "F.Cu") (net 8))
 (segment (start 88.9 71.755) (end 91.44 71.755) (width 0.4) (layer "F.Cu") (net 8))
 (segment (start 88.9 80.01) (end 88.9 71.755) (width 0.4) (layer "F.Cu") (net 8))
 (segment (start 87.63 81.28) (end 87.63 80.01) (width 0.4) (layer "F.Cu") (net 8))
 (segment (start 87.63 80.01) (end 88.9 80.01) (width 0.4) (layer "F.Cu") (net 8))
 (segment (start 91.44 68.58) (end 91.44 64.77) (width 0.4) (layer "B.Cu") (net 8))
 (segment (start 100.33 64.77) (end 100.33 58.42) (width 0.4) (layer "B.Cu") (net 8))
 (segment (start 91.44 64.77) (end 100.33 64.77) (width 0.4) (layer "B.Cu") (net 8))
 (segment (start 93.98 72.39) (end 93.98 68.58) (width 0.4) (layer "F.Cu") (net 7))
 (segment (start 91.44 72.39) (end 93.98 72.39) (width 0.4) (layer "F.Cu") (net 7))
 (segment (start 91.44 80.01) (end 91.44 72.39) (width 0.4) (layer "F.Cu") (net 7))
 (segment (start 90.17 81.28) (end 90.17 80.01) (width 0.4) (layer "F.Cu") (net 7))
 (segment (start 90.17 80.01) (end 91.44 80.01) (width 0.4) (layer "F.Cu") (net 7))
 (segment (start 105.41 66.167) (end 105.41 58.42) (width 0.4) (layer "B.Cu") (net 7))
 (segment (start 93.98 66.167) (end 105.41 66.167) (width 0.4) (layer "B.Cu") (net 7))
 (segment (start 93.98 68.58) (end 93.98 66.167) (width 0.4) (layer "B.Cu") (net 7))
 (segment (start 93.98 86.36) (end 93.98 86.36) (width 0.4) (layer "F.Cu") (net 5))
 (segment (start 95.25 74.803) (end 93.98 74.803) (width 0.4) (layer "F.Cu") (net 5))
 (segment (start 95.25 73.66) (end 95.25 74.803) (width 0.4) (layer "F.Cu") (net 5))
 (segment (start 93.98 80.899) (end 93.98 86.36) (width 0.4) (layer "F.Cu") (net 5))
 (segment (start 93.98 74.803) (end 93.98 80.899) (width 0.4) (layer "F.Cu") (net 5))
 (via (at 93.98 86.36) (size 0.8) (drill 0.4) (layers "F.Cu" "B.Cu") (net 5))
 (segment (start 62.865 86.36) (end 93.98 86.36) (width 0.4) (layer "B.Cu") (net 5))
 (segment (start 145.034 76.2) (end 145.034 86.36) (width 0.4) (layer "F.Cu") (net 17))
 (segment (start 145.034 86.36) (end 148.59 86.36) (width 0.4) (layer "F.Cu") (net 17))
 (via (at 145.034 76.2) (size 0.8) (drill 0.4) (layers "F.Cu" "B.Cu") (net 17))
 (segment (start 145.034 76.2) (end 145.034 76.2) (width 0.4) (layer "B.Cu") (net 17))
 (segment (start 140.335 73.66) (end 140.335 76.2) (width 0.4) (layer "B.Cu") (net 17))
 (segment (start 140.335 76.2) (end 145.034 76.2) (width 0.4) (layer "B.Cu") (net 17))
 (segment (start 137.795 73.66) (end 137.795 76.835) (width 0.4) (layer "B.Cu") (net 25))
 (segment (start 114.935 66.04) (end 114.935 58.42) (width 0.4) (layer "B.Cu") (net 25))
 (segment (start 126.365 72.009) (end 123.952 72.009) (width 0.4) (layer "B.Cu") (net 25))
 (segment (start 126.365 76.835) (end 126.365 72.009) (width 0.4) (layer "B.Cu") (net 25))
 (segment (start 123.952 72.009) (end 123.952 68.58) (width 0.4) (layer "B.Cu") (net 25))
 (segment (start 123.952 66.04) (end 114.935 66.04) (width 0.4) (layer "B.Cu") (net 25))
 (segment (start 137.795 76.835) (end 126.365 76.835) (width 0.4) (layer "B.Cu") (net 25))
 (segment (start 123.952 68.58) (end 123.952 66.04) (width 0.4) (layer "B.Cu") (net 25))
 (segment (start 135.255 75.438) (end 128.905 75.438) (width 0.4) (layer "B.Cu") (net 24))
 (segment (start 126.492 64.77) (end 120.015 64.77) (width 0.4) (layer "B.Cu") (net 24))
 (segment (start 128.905 71.12) (end 126.492 71.12) (width 0.4) (layer "B.Cu") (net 24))
 (segment (start 126.492 68.58) (end 126.492 64.77) (width 0.4) (layer "B.Cu") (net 24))
 (segment (start 120.015 64.77) (end 120.015 58.42) (width 0.4) (layer "B.Cu") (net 24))
 (segment (start 126.492 71.12) (end 126.492 68.58) (width 0.4) (layer "B.Cu") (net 24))
 (segment (start 135.255 73.66) (end 135.255 75.438) (width 0.4) (layer "B.Cu") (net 24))
 (segment (start 128.905 75.438) (end 128.905 71.12) (width 0.4) (layer "B.Cu") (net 24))
 (segment (start 129.032 68.58) (end 129.032 63.5) (width 0.4) (layer "B.Cu") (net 23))
 (segment (start 132.715 70.485) (end 129.032 70.485) (width 0.4) (layer "B.Cu") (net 23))
 (segment (start 132.715 73.66) (end 132.715 70.485) (width 0.4) (layer "B.Cu") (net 23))
 (segment (start 125.095 63.5) (end 125.095 58.42) (width 0.4) (layer "B.Cu") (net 23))
 (segment (start 129.032 63.5) (end 125.095 63.5) (width 0.4) (layer "B.Cu") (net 23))
 (segment (start 129.032 70.485) (end 129.032 68.58) (width 0.4) (layer "B.Cu") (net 23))
 (segment (start 130.175 69.723) (end 131.699 69.723) (width 0.4) (layer "F.Cu") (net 22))
 (segment (start 131.699 69.723) (end 131.699 68.707) (width 0.4) (layer "F.Cu") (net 22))
 (segment (start 130.175 73.66) (end 130.175 69.723) (width 0.4) (layer "F.Cu") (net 22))
 (segment (start 131.699 68.707) (end 131.572 68.58) (width 0.4) (layer "F.Cu") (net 22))
 (segment (start 130.175 62.23) (end 130.175 58.42) (width 0.4) (layer "B.Cu") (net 22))
 (segment (start 131.572 68.58) (end 131.572 62.23) (width 0.4) (layer "B.Cu") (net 22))
 (segment (start 131.572 62.23) (end 130.175 62.23) (width 0.4) (layer "B.Cu") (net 22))
 (segment (start 131.445 70.485) (end 134.112 70.485) (width 0.4) (layer "F.Cu") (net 21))
 (segment (start 131.445 80.01) (end 131.445 70.485) (width 0.4) (layer "F.Cu") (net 21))
 (segment (start 130.175 81.28) (end 130.175 80.01) (width 0.4) (layer "F.Cu") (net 21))
 (segment (start 130.175 80.01) (end 131.445 80.01) (width 0.4) (layer "F.Cu") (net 21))
 (segment (start 134.112 70.485) (end 134.112 68.58) (width 0.4) (layer "F.Cu") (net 21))
 (segment (start 134.112 68.58) (end 134.112 62.23) (width 0.4) (layer "B.Cu") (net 21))
 (segment (start 134.112 62.23) (end 135.255 62.23) (width 0.4) (layer "B.Cu") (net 21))
 (segment (start 135.255 62.23) (end 135.255 58.42) (width 0.4) (layer "B.Cu") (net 21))
 (segment (start 132.715 80.01) (end 133.985 80.01) (width 0.4) (layer "F.Cu") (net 20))
 (segment (start 133.985 71.12) (end 136.652 71.12) (width 0.4) (layer "F.Cu") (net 20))
 (segment (start 136.652 71.12) (end 136.652 68.58) (width 0.4) (layer "F.Cu") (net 20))
 (segment (start 133.985 80.01) (end 133.985 71.12) (width 0.4) (layer "F.Cu") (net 20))
 (segment (start 132.715 81.28) (end 132.715 80.01) (width 0.4) (layer "F.Cu") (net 20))
 (segment (start 136.652 63.5) (end 140.335 63.5) (width 0.4) (layer "B.Cu") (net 20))
 (segment (start 136.652 68.58) (end 136.652 63.5) (width 0.4) (layer "B.Cu") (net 20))
 (segment (start 140.335 63.5) (end 140.335 58.42) (width 0.4) (layer "B.Cu") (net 20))
 (segment (start 136.525 71.755) (end 139.192 71.755) (width 0.4) (layer "F.Cu") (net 19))
 (segment (start 139.192 71.755) (end 139.192 68.58) (width 0.4) (layer "F.Cu") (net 19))
 (segment (start 136.525 80.01) (end 136.525 71.755) (width 0.4) (layer "F.Cu") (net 19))
 (segment (start 135.255 80.01) (end 136.525 80.01) (width 0.4) (layer "F.Cu") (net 19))
 (segment (start 135.255 81.28) (end 135.255 80.01) (width 0.4) (layer "F.Cu") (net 19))
 (segment (start 145.415 64.77) (end 145.415 58.42) (width 0.4) (layer "B.Cu") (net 19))
 (segment (start 139.192 68.58) (end 139.192 64.77) (width 0.4) (layer "B.Cu") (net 19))
 (segment (start 139.192 64.77) (end 145.415 64.77) (width 0.4) (layer "B.Cu") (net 19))
 (segment (start 139.065 72.39) (end 141.732 72.39) (width 0.4) (layer "F.Cu") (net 18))
 (segment (start 141.732 72.39) (end 141.732 68.58) (width 0.4) (layer "F.Cu") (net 18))
 (segment (start 137.795 80.01) (end 139.065 80.01) (width 0.4) (layer "F.Cu") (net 18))
 (segment (start 137.795 81.28) (end 137.795 80.01) (width 0.4) (layer "F.Cu") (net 18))
 (segment (start 139.065 80.01) (end 139.065 72.39) (width 0.4) (layer "F.Cu") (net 18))
 (segment (start 141.732 66.04) (end 150.495 66.04) (width 0.4) (layer "B.Cu") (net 18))
 (segment (start 150.495 66.04) (end 150.495 58.42) (width 0.4) (layer "B.Cu") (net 18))
 (segment (start 141.732 68.58) (end 141.732 66.04) (width 0.4) (layer "B.Cu") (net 18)))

